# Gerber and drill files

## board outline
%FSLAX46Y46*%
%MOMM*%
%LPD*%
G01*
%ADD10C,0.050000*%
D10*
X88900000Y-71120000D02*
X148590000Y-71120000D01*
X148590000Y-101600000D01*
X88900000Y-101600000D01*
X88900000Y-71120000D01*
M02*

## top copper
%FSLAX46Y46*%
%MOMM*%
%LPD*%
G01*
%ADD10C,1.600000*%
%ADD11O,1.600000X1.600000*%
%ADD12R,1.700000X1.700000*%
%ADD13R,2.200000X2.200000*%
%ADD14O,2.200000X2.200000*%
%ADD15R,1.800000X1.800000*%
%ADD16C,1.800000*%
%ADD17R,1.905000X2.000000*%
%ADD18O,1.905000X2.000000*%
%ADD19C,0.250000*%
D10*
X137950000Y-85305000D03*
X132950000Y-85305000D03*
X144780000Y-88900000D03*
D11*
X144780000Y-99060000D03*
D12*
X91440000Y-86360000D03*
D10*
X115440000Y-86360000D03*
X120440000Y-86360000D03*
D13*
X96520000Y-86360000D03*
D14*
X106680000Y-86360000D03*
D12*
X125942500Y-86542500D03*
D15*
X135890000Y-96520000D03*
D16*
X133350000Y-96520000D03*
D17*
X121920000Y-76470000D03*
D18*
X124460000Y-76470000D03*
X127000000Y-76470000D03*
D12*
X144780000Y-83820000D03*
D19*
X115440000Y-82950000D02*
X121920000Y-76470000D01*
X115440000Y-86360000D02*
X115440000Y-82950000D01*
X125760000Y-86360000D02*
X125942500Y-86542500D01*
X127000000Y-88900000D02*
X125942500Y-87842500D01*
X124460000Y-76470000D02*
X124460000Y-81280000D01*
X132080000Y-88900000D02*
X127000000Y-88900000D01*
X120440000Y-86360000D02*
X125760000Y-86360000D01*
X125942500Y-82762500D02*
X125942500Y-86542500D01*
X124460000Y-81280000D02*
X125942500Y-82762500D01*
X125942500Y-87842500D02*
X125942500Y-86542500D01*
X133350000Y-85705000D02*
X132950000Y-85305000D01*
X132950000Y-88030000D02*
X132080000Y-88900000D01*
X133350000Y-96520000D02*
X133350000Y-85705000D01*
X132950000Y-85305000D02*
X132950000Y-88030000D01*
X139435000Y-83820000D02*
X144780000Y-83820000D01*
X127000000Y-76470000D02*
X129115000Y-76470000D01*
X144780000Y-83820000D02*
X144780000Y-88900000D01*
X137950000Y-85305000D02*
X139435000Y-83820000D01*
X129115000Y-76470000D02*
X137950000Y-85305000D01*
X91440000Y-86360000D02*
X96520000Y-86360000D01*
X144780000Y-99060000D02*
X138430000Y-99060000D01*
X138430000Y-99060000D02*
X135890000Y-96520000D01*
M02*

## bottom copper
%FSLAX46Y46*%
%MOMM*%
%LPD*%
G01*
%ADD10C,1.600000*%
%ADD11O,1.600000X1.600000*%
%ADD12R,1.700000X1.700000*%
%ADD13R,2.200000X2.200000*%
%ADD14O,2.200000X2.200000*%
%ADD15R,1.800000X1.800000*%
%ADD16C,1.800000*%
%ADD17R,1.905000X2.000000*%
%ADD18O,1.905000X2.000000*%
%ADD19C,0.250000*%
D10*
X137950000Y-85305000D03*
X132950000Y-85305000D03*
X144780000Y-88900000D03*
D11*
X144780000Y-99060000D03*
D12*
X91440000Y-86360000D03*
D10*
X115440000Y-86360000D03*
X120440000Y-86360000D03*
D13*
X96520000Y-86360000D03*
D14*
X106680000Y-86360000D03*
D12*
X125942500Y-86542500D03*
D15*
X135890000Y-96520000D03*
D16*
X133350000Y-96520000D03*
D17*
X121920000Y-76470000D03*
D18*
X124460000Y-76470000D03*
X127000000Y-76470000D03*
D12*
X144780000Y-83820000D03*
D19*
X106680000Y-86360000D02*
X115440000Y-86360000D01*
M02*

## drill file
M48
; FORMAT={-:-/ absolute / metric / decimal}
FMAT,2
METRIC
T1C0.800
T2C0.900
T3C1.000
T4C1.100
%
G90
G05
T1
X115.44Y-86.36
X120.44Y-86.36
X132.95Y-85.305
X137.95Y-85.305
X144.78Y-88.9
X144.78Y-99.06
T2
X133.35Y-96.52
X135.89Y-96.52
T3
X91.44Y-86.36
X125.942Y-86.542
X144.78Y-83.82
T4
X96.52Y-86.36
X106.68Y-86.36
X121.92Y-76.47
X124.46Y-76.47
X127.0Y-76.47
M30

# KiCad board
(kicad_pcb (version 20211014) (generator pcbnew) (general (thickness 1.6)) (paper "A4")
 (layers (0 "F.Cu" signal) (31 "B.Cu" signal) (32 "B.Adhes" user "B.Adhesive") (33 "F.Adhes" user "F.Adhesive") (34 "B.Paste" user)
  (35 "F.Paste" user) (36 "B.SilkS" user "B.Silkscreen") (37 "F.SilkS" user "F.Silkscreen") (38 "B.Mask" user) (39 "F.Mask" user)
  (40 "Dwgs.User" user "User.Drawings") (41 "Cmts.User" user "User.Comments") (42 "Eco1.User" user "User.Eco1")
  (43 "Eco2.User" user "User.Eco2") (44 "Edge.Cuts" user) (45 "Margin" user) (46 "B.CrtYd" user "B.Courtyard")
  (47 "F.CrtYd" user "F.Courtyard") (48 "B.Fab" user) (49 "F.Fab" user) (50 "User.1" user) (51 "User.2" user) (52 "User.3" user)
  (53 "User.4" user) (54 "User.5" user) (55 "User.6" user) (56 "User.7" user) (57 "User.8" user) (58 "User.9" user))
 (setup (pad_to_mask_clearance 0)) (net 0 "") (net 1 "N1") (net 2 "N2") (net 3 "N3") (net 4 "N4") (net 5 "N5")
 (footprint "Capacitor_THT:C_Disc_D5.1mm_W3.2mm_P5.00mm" (layer "F.Cu") (at 137.95 85.305 180)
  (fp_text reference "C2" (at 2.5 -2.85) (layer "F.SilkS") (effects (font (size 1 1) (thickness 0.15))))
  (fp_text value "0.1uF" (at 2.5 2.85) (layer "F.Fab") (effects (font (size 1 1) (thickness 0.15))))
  (pad "1" thru_hole circle (at 0 0 180) (size 1.6 1.6) (drill 0.8) (layers *.Cu *.Mask) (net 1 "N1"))
  (pad "2" thru_hole circle (at 5 0 180) (size 1.6 1.6) (drill 0.8) (layers *.Cu *.Mask) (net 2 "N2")))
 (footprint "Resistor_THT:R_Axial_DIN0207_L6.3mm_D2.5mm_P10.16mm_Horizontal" (layer "F.Cu") (at 144.78 88.9 -90)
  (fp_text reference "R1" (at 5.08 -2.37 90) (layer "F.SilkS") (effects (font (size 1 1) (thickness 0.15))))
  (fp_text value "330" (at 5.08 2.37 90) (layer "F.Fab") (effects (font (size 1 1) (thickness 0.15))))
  (pad "1" thru_hole circle (at 0 0 270) (size 1.6 1.6) (drill 0.8) (layers *.Cu *.Mask) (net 1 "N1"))
  (pad "2" thru_hole oval (at 10.16 0 270) (size 1.6 1.6) (drill 0.8) (layers *.Cu *.Mask) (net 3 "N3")))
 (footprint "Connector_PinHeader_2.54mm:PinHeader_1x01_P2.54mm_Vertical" (layer "F.Cu") (at 91.44 86.36)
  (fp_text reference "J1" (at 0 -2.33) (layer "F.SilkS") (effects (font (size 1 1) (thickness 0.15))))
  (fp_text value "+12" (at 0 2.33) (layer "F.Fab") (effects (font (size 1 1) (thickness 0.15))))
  (pad "1" thru_hole rect (at 0 0) (size 1.7 1.7) (drill 1) (layers *.Cu *.Mask) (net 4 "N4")))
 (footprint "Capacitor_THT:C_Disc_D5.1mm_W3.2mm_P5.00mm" (layer "F.Cu") (at 115.44 86.36)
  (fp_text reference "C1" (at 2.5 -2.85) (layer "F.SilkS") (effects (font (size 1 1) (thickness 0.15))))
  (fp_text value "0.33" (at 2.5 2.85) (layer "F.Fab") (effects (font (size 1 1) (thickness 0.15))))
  (pad "1" thru_hole circle (at 0 0) (size 1.6 1.6) (drill 0.8) (layers *.Cu *.Mask) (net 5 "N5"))
  (pad "2" thru_hole circle (at 5 0) (size 1.6 1.6) (drill 0.8) (layers *.Cu *.Mask) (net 2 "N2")))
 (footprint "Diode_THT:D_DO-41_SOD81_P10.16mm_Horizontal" (layer "F.Cu") (at 96.52 86.36)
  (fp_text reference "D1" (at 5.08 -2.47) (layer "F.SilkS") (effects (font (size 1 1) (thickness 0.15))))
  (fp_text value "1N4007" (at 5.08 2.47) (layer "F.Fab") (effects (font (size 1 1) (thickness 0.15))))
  (pad "1" thru_hole rect (at 0 0) (size 2.2 2.2) (drill 1.1) (layers *.Cu *.Mask) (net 4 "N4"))
  (pad "2" thru_hole oval (at 10.16 0) (size 2.2 2.2) (drill 1.1) (layers *.Cu *.Mask) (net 5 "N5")))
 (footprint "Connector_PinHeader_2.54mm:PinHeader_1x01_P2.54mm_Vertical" (layer "F.Cu") (at 125.9425 86.5425)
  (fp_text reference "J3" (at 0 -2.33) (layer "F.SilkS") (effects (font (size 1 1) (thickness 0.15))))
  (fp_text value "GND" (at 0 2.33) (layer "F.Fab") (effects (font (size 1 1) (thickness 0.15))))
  (pad "1" thru_hole rect (at 0 0) (size 1.7 1.7) (drill 1) (layers *.Cu *.Mask) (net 2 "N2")))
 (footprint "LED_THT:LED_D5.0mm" (layer "F.Cu") (at 135.89 96.52 180)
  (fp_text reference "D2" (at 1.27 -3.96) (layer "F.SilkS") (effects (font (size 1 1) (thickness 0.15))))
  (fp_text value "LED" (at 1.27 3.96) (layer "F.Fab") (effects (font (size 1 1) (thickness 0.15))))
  (pad "1" thru_hole rect (at 0 0 180) (size 1.8 1.8) (drill 0.9) (layers *.Cu *.Mask) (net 3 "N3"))
  (pad "2" thru_hole circle (at 2.54 0 180) (size 1.8 1.8) (drill 0.9) (layers *.Cu *.Mask) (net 2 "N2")))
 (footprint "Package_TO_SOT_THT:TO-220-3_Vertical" (layer "F.Cu") (at 121.92 76.47)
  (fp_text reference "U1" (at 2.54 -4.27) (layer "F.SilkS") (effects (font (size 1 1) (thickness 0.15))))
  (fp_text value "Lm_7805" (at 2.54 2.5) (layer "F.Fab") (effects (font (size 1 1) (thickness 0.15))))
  (pad "1" thru_hole rect (at 0 0) (size 1.905 2) (drill 1.1) (layers *.Cu *.Mask) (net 5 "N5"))
  (pad "2" thru_hole oval (at 2.54 0) (size 1.905 2) (drill 1.1) (layers *.Cu *.Mask) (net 2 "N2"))
  (pad "3" thru_hole oval (at 5.08 0) (size 1.905 2) (drill 1.1) (layers *.Cu *.Mask) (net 1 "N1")))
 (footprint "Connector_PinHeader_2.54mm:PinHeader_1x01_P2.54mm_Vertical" (layer "F.Cu") (at 144.78 83.82)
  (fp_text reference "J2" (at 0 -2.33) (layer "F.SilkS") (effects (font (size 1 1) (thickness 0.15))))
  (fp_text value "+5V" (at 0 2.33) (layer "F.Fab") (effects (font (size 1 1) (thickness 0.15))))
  (pad "1" thru_hole rect (at 0 0) (size 1.7 1.7) (drill 1) (layers *.Cu *.Mask) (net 1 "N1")))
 (gr_rect (start 148.59 101.6) (end 148.59 101.6) (layer "Edge.Cuts") (width 0.05) (fill none))
 (gr_rect (start 88.9 71.12) (end 148.59 101.6) (layer "Edge.Cuts") (width 0.05) (fill none))
 (segment (start 115.44 82.95) (end 121.92 76.47) (width 0.25) (layer "F.Cu") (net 5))
 (segment (start 115.44 86.36) (end 115.44 82.95) (width 0.25) (layer "F.Cu") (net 5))
 (segment (start 106.68 86.36) (end 115.44 86.36) (width 0.25) (layer "B.Cu") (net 5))
 (segment (start 125.76 86.36) (end 125.9425 86.5425) (width 0.25) (layer "F.Cu") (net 2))
 (segment (start 127 88.9) (end 125.9425 87.8425) (width 0.25) (layer "F.Cu") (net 2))
 (segment (start 124.46 76.47) (end 124.46 81.28) (width 0.25) (layer "F.Cu") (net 2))
 (segment (start 132.08 88.9) (end 127 88.9) (width 0.25) (layer "F.Cu") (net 2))
 (segment (start 120.44 86.36) (end 125.76 86.36) (width 0.25) (layer "F.Cu") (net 2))
 (segment (start 125.9425 82.7625) (end 125.9425 86.5425) (width 0.25) (layer "F.Cu") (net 2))
 (segment (start 124.46 81.28) (end 125.9425 82.7625) (width 0.25) (layer "F.Cu") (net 2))
 (segment (start 125.9425 87.8425) (end 125.9425 86.5425) (width 0.25) (layer "F.Cu") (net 2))
 (segment (start 133.35 85.705) (end 132.95 85.305) (width 0.25) (layer "F.Cu") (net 2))
 (segment (start 132.95 88.03) (end 132.08 88.9) (width 0.25) (layer "F.Cu") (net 2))
 (segment (start 133.35 96.52) (end 133.35 85.705) (width 0.25) (layer "F.Cu") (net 2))
 (segment (start 132.95 85.305) (end 132.95 88.03) (width 0.25) (layer "F.Cu") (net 2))
 (segment (start 139.435 83.82) (end 144.78 83.82) (width 0.25) (layer "F.Cu") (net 1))
 (segment (start 127 76.47) (end 129.115 76.47) (width 0.25) (layer "F.Cu") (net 1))
 (segment (start 144.78 83.82) (end 144.78 88.9) (width 0.25) (layer "F.Cu") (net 1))
 (segment (start 137.95 85.305) (end 139.435 83.82) (width 0.25) (layer "F.Cu") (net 1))
 (segment (start 129.115 76.47) (end 137.95 85.305) (width 0.25) (layer "F.Cu") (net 1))
 (segment (start 91.44 86.36) (end 96.52 86.36) (width 0.25) (layer "F.Cu") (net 4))
 (segment (start 144.78 99.06) (end 138.43 99.06) (width 0.25) (layer "F.Cu") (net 3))
 (segment (start 138.43 99.06) (end 135.89 96.52) (width 0.25) (layer "F.Cu") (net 3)))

